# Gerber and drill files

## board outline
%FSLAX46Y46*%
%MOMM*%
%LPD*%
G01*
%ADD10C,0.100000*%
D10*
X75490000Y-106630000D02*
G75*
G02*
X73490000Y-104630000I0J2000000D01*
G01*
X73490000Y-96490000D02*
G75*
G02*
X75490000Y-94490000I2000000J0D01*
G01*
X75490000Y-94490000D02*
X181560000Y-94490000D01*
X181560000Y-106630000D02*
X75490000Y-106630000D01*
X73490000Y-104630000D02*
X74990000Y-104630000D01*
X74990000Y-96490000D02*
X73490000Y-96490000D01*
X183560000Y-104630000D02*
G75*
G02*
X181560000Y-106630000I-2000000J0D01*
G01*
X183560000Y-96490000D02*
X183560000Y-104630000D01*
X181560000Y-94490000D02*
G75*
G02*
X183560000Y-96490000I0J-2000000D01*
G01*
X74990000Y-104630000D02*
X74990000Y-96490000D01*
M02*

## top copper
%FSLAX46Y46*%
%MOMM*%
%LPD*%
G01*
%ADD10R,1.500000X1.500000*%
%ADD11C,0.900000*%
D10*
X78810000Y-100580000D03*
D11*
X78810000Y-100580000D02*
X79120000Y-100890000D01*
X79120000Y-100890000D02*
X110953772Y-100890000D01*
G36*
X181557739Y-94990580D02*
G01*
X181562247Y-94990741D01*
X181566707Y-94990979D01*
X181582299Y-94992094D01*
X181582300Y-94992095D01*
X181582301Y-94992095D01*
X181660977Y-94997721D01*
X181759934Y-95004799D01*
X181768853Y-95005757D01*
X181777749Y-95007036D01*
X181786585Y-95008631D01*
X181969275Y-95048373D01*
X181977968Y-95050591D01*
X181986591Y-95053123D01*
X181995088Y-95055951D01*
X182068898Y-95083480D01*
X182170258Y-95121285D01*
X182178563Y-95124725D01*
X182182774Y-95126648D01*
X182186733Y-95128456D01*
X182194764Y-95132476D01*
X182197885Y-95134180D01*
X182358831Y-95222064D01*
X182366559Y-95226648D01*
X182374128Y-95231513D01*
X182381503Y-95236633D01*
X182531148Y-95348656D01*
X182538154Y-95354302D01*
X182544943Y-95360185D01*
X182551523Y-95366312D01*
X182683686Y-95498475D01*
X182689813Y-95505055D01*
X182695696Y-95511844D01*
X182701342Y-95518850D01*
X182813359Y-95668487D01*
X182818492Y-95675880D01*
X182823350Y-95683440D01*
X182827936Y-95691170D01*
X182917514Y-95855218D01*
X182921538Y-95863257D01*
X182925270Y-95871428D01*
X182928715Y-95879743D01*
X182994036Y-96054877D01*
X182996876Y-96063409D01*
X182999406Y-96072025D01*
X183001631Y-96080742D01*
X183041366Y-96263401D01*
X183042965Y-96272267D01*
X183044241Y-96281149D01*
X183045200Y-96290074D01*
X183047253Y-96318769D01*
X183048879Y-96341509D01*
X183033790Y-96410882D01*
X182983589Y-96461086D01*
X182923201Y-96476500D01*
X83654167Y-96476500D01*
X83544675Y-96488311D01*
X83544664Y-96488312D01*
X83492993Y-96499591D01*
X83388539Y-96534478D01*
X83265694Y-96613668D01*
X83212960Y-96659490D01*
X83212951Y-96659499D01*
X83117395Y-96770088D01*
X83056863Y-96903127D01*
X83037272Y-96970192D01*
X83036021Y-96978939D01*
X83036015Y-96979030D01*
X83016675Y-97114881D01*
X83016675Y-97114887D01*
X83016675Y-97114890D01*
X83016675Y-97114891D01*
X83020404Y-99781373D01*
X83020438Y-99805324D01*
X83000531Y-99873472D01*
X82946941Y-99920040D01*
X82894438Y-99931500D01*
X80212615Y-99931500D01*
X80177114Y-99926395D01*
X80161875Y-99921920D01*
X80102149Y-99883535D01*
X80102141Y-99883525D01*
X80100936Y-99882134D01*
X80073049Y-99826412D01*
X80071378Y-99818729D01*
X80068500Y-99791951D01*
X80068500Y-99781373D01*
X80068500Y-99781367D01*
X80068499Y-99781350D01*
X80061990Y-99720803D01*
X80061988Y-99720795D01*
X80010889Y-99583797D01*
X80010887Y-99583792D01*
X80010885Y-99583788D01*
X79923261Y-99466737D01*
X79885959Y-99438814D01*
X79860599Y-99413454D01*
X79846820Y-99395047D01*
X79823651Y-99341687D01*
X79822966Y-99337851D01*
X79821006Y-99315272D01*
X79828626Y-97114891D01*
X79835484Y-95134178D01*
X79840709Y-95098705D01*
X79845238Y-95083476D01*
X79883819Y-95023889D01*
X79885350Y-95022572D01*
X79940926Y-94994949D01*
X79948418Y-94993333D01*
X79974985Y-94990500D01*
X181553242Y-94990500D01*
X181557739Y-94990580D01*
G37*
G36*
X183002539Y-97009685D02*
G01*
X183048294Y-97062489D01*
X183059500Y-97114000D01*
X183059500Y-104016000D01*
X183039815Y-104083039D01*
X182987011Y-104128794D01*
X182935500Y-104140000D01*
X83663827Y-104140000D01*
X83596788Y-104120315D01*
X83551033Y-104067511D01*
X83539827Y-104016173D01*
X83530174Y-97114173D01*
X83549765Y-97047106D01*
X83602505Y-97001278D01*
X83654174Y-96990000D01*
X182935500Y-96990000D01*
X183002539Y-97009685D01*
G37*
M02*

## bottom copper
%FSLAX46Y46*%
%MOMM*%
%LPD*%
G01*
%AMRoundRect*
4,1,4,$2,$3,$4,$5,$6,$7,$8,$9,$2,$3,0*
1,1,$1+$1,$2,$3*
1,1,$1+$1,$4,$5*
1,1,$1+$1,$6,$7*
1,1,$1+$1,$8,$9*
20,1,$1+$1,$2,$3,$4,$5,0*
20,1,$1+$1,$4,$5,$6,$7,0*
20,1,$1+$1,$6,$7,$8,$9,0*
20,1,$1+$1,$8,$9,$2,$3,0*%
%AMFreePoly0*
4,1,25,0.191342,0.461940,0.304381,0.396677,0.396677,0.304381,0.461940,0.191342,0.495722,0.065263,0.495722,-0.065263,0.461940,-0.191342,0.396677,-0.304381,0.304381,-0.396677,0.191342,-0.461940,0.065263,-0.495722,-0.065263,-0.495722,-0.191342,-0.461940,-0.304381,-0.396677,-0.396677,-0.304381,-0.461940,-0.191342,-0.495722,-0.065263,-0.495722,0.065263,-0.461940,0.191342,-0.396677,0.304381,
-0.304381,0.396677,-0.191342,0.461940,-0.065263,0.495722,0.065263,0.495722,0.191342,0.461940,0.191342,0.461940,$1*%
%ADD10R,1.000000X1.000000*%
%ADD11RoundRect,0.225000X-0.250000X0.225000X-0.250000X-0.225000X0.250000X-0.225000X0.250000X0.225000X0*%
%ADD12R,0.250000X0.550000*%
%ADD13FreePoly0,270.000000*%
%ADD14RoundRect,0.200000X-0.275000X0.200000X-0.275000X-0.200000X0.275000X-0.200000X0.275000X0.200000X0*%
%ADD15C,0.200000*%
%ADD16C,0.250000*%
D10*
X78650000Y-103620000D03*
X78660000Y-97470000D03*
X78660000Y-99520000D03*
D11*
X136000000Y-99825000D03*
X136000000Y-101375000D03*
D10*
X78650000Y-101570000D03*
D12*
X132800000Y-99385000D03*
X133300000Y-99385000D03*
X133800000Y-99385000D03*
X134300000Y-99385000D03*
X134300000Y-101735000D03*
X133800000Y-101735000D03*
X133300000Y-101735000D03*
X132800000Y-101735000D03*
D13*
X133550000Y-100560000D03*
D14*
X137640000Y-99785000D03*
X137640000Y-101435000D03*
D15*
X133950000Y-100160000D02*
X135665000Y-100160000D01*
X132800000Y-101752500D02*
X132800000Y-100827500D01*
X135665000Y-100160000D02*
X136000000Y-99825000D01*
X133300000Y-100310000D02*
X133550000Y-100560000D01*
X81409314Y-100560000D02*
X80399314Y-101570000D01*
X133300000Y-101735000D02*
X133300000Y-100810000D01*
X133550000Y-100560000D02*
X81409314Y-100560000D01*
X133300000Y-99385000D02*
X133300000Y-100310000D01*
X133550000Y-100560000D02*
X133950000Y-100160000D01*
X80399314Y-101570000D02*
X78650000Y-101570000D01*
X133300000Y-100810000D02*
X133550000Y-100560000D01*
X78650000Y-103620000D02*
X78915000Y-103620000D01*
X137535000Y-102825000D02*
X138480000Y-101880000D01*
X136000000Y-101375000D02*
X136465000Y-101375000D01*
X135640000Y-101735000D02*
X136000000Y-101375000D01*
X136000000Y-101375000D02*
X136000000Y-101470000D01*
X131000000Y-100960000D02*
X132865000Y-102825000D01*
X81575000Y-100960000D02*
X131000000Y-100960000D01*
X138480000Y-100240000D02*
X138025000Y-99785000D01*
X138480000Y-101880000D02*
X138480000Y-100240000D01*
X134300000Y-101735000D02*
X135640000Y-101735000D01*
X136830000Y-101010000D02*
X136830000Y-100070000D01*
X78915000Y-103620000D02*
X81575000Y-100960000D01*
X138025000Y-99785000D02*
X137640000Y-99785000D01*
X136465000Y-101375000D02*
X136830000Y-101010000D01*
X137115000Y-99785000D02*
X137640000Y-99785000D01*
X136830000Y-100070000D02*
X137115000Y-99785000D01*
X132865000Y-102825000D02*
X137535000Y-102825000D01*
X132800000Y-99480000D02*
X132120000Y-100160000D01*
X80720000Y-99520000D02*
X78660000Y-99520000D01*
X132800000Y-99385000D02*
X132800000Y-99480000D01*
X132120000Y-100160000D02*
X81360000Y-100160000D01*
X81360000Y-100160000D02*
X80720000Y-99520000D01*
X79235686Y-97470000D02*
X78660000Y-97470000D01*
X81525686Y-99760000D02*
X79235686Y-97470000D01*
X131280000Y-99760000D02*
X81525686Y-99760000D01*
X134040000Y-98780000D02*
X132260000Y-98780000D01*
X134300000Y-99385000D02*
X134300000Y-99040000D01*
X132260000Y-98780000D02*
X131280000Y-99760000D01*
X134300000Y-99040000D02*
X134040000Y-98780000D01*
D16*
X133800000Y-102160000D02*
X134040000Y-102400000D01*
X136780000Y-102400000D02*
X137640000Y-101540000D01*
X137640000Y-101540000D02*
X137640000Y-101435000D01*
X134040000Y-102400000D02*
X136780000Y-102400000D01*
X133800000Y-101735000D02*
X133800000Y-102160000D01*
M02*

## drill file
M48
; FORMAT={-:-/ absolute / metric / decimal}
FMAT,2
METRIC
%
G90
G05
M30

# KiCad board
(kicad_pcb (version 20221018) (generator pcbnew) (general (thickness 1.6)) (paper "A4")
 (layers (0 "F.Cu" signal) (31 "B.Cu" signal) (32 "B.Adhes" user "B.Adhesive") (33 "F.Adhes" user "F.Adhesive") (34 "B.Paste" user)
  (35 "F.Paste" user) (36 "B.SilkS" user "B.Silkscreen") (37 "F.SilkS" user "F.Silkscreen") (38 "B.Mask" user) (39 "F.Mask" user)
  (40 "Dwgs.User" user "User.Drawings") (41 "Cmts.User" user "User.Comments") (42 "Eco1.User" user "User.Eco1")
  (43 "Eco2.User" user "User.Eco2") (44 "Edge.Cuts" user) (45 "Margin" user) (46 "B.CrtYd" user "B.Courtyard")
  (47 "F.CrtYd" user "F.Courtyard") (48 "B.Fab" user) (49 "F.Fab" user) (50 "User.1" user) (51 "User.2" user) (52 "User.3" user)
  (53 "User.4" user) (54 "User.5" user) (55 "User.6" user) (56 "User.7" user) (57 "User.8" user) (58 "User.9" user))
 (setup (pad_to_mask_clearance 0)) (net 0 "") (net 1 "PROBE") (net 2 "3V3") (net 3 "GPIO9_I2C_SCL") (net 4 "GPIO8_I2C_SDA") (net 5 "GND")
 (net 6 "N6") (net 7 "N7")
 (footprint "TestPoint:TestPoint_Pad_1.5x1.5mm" (layer "F.Cu") (at 78.81 100.58)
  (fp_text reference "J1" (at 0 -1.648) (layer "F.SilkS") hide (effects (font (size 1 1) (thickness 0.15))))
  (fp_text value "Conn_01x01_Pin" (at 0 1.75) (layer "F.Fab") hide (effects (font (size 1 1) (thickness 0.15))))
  (pad "1" smd rect (at 0 0) (size 1.5 1.5) (layers "F.Cu" "F.Mask") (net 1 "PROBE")))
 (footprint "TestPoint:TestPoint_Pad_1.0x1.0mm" (layer "B.Cu") (at 78.65 103.62 180)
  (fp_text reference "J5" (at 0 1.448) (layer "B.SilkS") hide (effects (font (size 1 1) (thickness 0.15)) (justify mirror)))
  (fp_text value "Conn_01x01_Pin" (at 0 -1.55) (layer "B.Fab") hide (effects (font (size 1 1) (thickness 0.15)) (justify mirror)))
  (pad "1" smd rect (at 0 0 180) (size 1 1) (layers "B.Cu" "B.Mask") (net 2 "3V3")))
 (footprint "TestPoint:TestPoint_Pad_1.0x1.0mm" (layer "B.Cu") (at 78.66 97.47 180)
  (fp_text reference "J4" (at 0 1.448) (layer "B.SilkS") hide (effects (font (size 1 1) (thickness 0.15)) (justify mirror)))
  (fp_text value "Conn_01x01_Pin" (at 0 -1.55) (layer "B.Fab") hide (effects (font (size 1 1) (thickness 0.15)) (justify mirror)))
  (pad "1" smd rect (at 0 0 180) (size 1 1) (layers "B.Cu" "B.Mask") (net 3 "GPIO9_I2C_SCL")))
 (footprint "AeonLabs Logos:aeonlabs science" (layer "B.Cu") (at 174.189702 103.971553 180)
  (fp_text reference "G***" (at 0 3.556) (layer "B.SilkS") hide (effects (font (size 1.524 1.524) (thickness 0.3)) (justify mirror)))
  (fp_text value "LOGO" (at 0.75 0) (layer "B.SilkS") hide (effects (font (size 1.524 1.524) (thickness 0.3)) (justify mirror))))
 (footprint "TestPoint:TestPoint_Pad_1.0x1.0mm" (layer "B.Cu") (at 78.66 99.52 180)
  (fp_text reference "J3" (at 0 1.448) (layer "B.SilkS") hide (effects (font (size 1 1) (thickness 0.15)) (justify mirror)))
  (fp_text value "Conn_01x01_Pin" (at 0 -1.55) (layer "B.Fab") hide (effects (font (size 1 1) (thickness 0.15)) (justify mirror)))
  (pad "1" smd rect (at 0 0 180) (size 1 1) (layers "B.Cu" "B.Mask") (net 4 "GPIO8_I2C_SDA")))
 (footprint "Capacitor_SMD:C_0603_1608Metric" (layer "B.Cu") (at 136 100.6 -90)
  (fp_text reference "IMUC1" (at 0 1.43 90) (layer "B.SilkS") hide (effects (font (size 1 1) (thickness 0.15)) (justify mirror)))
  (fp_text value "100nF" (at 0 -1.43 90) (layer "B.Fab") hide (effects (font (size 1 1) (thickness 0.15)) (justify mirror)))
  (pad "1" smd roundrect (at -0.775 0 270) (size 0.9 0.95) (layers "B.Cu" "B.Paste" "B.Mask") (roundrect_rratio 0.25) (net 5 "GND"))
  (pad "2" smd roundrect (at 0.775 0 270) (size 0.9 0.95) (layers "B.Cu" "B.Paste" "B.Mask") (roundrect_rratio 0.25) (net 2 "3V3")))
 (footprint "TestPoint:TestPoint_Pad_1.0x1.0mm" (layer "B.Cu") (at 78.65 101.57 180)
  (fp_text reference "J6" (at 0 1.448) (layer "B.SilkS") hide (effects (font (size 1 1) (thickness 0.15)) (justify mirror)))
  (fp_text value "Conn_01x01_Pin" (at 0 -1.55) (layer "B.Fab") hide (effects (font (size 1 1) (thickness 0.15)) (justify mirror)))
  (pad "1" smd rect (at 0 0 180) (size 1 1) (layers "B.Cu" "B.Mask") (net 5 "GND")))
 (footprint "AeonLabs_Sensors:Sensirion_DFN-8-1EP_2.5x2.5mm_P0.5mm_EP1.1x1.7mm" (layer "B.Cu") (at 133.55 100.56 -90)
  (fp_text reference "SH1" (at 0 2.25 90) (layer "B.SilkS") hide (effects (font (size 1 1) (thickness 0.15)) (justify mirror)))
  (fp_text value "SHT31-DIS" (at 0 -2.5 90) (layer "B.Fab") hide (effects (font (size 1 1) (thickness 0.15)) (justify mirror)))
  (pad "" smd custom (at 0 0 270) (size 0.9 0.9) (layers "B.Paste") (zone_connect 0) (thermal_bridge_angle 45)
   (options (clearance outline) (anchor rect)) (primitives))
  (pad "1" smd rect (at -1.175 0.75 270) (size 0.55 0.25) (layers "B.Cu" "B.Paste" "B.Mask") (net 4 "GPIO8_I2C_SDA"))
  (pad "2" smd rect (at -1.175 0.25 270) (size 0.55 0.25) (layers "B.Cu" "B.Paste" "B.Mask") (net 5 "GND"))
  (pad "3" smd rect (at -1.175 -0.25 270) (size 0.55 0.25) (layers "B.Cu" "B.Paste" "B.Mask") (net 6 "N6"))
  (pad "4" smd rect (at -1.175 -0.75 90) (size 0.55 0.25) (layers "B.Cu" "B.Paste" "B.Mask") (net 3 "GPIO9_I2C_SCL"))
  (pad "5" smd rect (at 1.175 -0.75 270) (size 0.55 0.25) (layers "B.Cu" "B.Paste" "B.Mask") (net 2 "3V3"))
  (pad "6" smd rect (at 1.175 -0.25 270) (size 0.55 0.25) (layers "B.Cu" "B.Paste" "B.Mask") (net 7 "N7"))
  (pad "7" smd rect (at 1.175 0.25 270) (size 0.55 0.25) (layers "B.Cu" "B.Paste" "B.Mask") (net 5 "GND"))
  (pad "8" smd rect (at 1.175 0.75 270) (size 0.55 0.25) (layers "B.Cu" "B.Paste" "B.Mask") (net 5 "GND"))
  (pad "9" smd custom (at 0 0 270) (size 1 1) (layers "B.Cu" "B.Mask") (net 5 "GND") (zone_connect 0)
   (options (clearance outline) (anchor circle)) (primitives)))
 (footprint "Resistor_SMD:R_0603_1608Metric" (layer "B.Cu") (at 137.64 100.61 -90)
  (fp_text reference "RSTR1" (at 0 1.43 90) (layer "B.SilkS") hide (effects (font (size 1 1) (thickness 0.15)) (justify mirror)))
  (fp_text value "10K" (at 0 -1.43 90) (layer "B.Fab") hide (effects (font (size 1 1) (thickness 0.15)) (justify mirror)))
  (pad "1" smd roundrect (at -0.825 0 270) (size 0.8 0.95) (layers "B.Cu" "B.Paste" "B.Mask") (roundrect_rratio 0.25) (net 2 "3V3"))
  (pad "2" smd roundrect (at 0.825 0 270) (size 0.8 0.95) (layers "B.Cu" "B.Paste" "B.Mask") (roundrect_rratio 0.25) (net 7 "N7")))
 (gr_arc (start 75.49 106.63) (mid 74.075786 106.044214) (end 73.49 104.63) (stroke (width 0.1) (type default)) (layer "Edge.Cuts"))
 (gr_arc (start 73.49 96.49) (mid 74.075786 95.075786) (end 75.49 94.49) (stroke (width 0.1) (type default)) (layer "Edge.Cuts"))
 (gr_line (start 75.49 94.49) (end 181.56 94.49) (stroke (width 0.1) (type default)) (layer "Edge.Cuts"))
 (gr_line (start 181.56 106.63) (end 75.49 106.63) (stroke (width 0.1) (type default)) (layer "Edge.Cuts"))
 (gr_line (start 73.49 104.63) (end 74.99 104.63) (stroke (width 0.1) (type default)) (layer "Edge.Cuts"))
 (gr_line (start 74.99 96.49) (end 73.49 96.49) (stroke (width 0.1) (type default)) (layer "Edge.Cuts"))
 (gr_arc (start 183.56 104.63) (mid 182.974214 106.044214) (end 181.56 106.63) (stroke (width 0.1) (type default)) (layer "Edge.Cuts"))
 (gr_line (start 183.56 96.49) (end 183.56 104.63) (stroke (width 0.1) (type default)) (layer "Edge.Cuts"))
 (gr_arc (start 181.56 94.49) (mid 182.974214 95.075786) (end 183.56 96.49) (stroke (width 0.1) (type default)) (layer "Edge.Cuts"))
 (gr_line (start 74.99 104.63) (end 74.99 96.49) (stroke (width 0.1) (type default)) (layer "Edge.Cuts"))
 (segment (start 78.81 100.58) (end 79.12 100.89) (width 0.9) (layer "F.Cu") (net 1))
 (segment (start 79.12 100.89) (end 110.953772 100.89) (width 0.9) (layer "F.Cu") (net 1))
 (segment (start 133.95 100.16) (end 135.665 100.16) (width 0.2) (layer "B.Cu") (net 5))
 (segment (start 132.8 101.7525) (end 132.8 100.8275) (width 0.2) (layer "B.Cu") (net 5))
 (segment (start 135.665 100.16) (end 136 99.825) (width 0.2) (layer "B.Cu") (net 5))
 (segment (start 133.3 100.31) (end 133.55 100.56) (width 0.2) (layer "B.Cu") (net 5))
 (segment (start 81.409314 100.56) (end 80.399314 101.57) (width 0.2) (layer "B.Cu") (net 5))
 (segment (start 133.3 101.735) (end 133.3 100.81) (width 0.2) (layer "B.Cu") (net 5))
 (segment (start 133.55 100.56) (end 81.409314 100.56) (width 0.2) (layer "B.Cu") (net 5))
 (segment (start 133.3 99.385) (end 133.3 100.31) (width 0.2) (layer "B.Cu") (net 5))
 (segment (start 133.55 100.56) (end 133.95 100.16) (width 0.2) (layer "B.Cu") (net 5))
 (segment (start 80.399314 101.57) (end 78.65 101.57) (width 0.2) (layer "B.Cu") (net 5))
 (segment (start 133.3 100.81) (end 133.55 100.56) (width 0.2) (layer "B.Cu") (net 5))
 (segment (start 78.65 103.62) (end 78.915 103.62) (width 0.2) (layer "B.Cu") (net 2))
 (segment (start 137.535 102.825) (end 138.48 101.88) (width 0.2) (layer "B.Cu") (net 2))
 (segment (start 136 101.375) (end 136.465 101.375) (width 0.2) (layer "B.Cu") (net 2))
 (segment (start 135.64 101.735) (end 136 101.375) (width 0.2) (layer "B.Cu") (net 2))
 (segment (start 136 101.375) (end 136 101.47) (width 0.2) (layer "B.Cu") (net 2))
 (segment (start 131 100.96) (end 132.865 102.825) (width 0.2) (layer "B.Cu") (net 2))
 (segment (start 81.575 100.96) (end 131 100.96) (width 0.2) (layer "B.Cu") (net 2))
 (segment (start 138.48 100.24) (end 138.025 99.785) (width 0.2) (layer "B.Cu") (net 2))
 (segment (start 138.48 101.88) (end 138.48 100.24) (width 0.2) (layer "B.Cu") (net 2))
 (segment (start 134.3 101.735) (end 135.64 101.735) (width 0.2) (layer "B.Cu") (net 2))
 (segment (start 136.83 101.01) (end 136.83 100.07) (width 0.2) (layer "B.Cu") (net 2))
 (segment (start 78.915 103.62) (end 81.575 100.96) (width 0.2) (layer "B.Cu") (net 2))
 (segment (start 138.025 99.785) (end 137.64 99.785) (width 0.2) (layer "B.Cu") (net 2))
 (segment (start 136.465 101.375) (end 136.83 101.01) (width 0.2) (layer "B.Cu") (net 2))
 (segment (start 137.115 99.785) (end 137.64 99.785) (width 0.2) (layer "B.Cu") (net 2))
 (segment (start 136.83 100.07) (end 137.115 99.785) (width 0.2) (layer "B.Cu") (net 2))
 (segment (start 132.865 102.825) (end 137.535 102.825) (width 0.2) (layer "B.Cu") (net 2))
 (segment (start 132.8 99.48) (end 132.12 100.16) (width 0.2) (layer "B.Cu") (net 4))
 (segment (start 80.72 99.52) (end 78.66 99.52) (width 0.2) (layer "B.Cu") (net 4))
 (segment (start 132.8 99.385) (end 132.8 99.48) (width 0.2) (layer "B.Cu") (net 4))
 (segment (start 132.12 100.16) (end 81.36 100.16) (width 0.2) (layer "B.Cu") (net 4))
 (segment (start 81.36 100.16) (end 80.72 99.52) (width 0.2) (layer "B.Cu") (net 4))
 (segment (start 79.235686 97.47) (end 78.66 97.47) (width 0.2) (layer "B.Cu") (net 3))
 (segment (start 81.525686 99.76) (end 79.235686 97.47) (width 0.2) (layer "B.Cu") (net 3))
 (segment (start 131.28 99.76) (end 81.525686 99.76) (width 0.2) (layer "B.Cu") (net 3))
 (segment (start 134.04 98.78) (end 132.26 98.78) (width 0.2) (layer "B.Cu") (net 3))
 (segment (start 134.3 99.385) (end 134.3 99.04) (width 0.2) (layer "B.Cu") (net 3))
 (segment (start 132.26 98.78) (end 131.28 99.76) (width 0.2) (layer "B.Cu") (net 3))
 (segment (start 134.3 99.04) (end 134.04 98.78) (width 0.2) (layer "B.Cu") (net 3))
 (segment (start 133.8 102.16) (end 134.04 102.4) (width 0.25) (layer "B.Cu") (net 7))
 (segment (start 136.78 102.4) (end 137.64 101.54) (width 0.25) (layer "B.Cu") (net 7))
 (segment (start 137.64 101.54) (end 137.64 101.435) (width 0.25) (layer "B.Cu") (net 7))
 (segment (start 134.04 102.4) (end 136.78 102.4) (width 0.25) (layer "B.Cu") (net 7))
 (segment (start 133.8 101.735) (end 133.8 102.16) (width 0.25) (layer "B.Cu") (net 7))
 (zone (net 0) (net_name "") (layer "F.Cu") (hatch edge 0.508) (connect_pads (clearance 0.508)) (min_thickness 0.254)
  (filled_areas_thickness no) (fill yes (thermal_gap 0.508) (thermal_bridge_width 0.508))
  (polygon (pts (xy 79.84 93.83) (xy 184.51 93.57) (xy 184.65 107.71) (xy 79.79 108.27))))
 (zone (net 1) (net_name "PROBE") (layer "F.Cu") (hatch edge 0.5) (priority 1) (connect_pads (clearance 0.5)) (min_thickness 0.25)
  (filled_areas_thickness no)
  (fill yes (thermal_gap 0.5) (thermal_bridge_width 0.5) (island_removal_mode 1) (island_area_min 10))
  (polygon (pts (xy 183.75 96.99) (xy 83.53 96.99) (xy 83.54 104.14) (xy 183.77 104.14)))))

